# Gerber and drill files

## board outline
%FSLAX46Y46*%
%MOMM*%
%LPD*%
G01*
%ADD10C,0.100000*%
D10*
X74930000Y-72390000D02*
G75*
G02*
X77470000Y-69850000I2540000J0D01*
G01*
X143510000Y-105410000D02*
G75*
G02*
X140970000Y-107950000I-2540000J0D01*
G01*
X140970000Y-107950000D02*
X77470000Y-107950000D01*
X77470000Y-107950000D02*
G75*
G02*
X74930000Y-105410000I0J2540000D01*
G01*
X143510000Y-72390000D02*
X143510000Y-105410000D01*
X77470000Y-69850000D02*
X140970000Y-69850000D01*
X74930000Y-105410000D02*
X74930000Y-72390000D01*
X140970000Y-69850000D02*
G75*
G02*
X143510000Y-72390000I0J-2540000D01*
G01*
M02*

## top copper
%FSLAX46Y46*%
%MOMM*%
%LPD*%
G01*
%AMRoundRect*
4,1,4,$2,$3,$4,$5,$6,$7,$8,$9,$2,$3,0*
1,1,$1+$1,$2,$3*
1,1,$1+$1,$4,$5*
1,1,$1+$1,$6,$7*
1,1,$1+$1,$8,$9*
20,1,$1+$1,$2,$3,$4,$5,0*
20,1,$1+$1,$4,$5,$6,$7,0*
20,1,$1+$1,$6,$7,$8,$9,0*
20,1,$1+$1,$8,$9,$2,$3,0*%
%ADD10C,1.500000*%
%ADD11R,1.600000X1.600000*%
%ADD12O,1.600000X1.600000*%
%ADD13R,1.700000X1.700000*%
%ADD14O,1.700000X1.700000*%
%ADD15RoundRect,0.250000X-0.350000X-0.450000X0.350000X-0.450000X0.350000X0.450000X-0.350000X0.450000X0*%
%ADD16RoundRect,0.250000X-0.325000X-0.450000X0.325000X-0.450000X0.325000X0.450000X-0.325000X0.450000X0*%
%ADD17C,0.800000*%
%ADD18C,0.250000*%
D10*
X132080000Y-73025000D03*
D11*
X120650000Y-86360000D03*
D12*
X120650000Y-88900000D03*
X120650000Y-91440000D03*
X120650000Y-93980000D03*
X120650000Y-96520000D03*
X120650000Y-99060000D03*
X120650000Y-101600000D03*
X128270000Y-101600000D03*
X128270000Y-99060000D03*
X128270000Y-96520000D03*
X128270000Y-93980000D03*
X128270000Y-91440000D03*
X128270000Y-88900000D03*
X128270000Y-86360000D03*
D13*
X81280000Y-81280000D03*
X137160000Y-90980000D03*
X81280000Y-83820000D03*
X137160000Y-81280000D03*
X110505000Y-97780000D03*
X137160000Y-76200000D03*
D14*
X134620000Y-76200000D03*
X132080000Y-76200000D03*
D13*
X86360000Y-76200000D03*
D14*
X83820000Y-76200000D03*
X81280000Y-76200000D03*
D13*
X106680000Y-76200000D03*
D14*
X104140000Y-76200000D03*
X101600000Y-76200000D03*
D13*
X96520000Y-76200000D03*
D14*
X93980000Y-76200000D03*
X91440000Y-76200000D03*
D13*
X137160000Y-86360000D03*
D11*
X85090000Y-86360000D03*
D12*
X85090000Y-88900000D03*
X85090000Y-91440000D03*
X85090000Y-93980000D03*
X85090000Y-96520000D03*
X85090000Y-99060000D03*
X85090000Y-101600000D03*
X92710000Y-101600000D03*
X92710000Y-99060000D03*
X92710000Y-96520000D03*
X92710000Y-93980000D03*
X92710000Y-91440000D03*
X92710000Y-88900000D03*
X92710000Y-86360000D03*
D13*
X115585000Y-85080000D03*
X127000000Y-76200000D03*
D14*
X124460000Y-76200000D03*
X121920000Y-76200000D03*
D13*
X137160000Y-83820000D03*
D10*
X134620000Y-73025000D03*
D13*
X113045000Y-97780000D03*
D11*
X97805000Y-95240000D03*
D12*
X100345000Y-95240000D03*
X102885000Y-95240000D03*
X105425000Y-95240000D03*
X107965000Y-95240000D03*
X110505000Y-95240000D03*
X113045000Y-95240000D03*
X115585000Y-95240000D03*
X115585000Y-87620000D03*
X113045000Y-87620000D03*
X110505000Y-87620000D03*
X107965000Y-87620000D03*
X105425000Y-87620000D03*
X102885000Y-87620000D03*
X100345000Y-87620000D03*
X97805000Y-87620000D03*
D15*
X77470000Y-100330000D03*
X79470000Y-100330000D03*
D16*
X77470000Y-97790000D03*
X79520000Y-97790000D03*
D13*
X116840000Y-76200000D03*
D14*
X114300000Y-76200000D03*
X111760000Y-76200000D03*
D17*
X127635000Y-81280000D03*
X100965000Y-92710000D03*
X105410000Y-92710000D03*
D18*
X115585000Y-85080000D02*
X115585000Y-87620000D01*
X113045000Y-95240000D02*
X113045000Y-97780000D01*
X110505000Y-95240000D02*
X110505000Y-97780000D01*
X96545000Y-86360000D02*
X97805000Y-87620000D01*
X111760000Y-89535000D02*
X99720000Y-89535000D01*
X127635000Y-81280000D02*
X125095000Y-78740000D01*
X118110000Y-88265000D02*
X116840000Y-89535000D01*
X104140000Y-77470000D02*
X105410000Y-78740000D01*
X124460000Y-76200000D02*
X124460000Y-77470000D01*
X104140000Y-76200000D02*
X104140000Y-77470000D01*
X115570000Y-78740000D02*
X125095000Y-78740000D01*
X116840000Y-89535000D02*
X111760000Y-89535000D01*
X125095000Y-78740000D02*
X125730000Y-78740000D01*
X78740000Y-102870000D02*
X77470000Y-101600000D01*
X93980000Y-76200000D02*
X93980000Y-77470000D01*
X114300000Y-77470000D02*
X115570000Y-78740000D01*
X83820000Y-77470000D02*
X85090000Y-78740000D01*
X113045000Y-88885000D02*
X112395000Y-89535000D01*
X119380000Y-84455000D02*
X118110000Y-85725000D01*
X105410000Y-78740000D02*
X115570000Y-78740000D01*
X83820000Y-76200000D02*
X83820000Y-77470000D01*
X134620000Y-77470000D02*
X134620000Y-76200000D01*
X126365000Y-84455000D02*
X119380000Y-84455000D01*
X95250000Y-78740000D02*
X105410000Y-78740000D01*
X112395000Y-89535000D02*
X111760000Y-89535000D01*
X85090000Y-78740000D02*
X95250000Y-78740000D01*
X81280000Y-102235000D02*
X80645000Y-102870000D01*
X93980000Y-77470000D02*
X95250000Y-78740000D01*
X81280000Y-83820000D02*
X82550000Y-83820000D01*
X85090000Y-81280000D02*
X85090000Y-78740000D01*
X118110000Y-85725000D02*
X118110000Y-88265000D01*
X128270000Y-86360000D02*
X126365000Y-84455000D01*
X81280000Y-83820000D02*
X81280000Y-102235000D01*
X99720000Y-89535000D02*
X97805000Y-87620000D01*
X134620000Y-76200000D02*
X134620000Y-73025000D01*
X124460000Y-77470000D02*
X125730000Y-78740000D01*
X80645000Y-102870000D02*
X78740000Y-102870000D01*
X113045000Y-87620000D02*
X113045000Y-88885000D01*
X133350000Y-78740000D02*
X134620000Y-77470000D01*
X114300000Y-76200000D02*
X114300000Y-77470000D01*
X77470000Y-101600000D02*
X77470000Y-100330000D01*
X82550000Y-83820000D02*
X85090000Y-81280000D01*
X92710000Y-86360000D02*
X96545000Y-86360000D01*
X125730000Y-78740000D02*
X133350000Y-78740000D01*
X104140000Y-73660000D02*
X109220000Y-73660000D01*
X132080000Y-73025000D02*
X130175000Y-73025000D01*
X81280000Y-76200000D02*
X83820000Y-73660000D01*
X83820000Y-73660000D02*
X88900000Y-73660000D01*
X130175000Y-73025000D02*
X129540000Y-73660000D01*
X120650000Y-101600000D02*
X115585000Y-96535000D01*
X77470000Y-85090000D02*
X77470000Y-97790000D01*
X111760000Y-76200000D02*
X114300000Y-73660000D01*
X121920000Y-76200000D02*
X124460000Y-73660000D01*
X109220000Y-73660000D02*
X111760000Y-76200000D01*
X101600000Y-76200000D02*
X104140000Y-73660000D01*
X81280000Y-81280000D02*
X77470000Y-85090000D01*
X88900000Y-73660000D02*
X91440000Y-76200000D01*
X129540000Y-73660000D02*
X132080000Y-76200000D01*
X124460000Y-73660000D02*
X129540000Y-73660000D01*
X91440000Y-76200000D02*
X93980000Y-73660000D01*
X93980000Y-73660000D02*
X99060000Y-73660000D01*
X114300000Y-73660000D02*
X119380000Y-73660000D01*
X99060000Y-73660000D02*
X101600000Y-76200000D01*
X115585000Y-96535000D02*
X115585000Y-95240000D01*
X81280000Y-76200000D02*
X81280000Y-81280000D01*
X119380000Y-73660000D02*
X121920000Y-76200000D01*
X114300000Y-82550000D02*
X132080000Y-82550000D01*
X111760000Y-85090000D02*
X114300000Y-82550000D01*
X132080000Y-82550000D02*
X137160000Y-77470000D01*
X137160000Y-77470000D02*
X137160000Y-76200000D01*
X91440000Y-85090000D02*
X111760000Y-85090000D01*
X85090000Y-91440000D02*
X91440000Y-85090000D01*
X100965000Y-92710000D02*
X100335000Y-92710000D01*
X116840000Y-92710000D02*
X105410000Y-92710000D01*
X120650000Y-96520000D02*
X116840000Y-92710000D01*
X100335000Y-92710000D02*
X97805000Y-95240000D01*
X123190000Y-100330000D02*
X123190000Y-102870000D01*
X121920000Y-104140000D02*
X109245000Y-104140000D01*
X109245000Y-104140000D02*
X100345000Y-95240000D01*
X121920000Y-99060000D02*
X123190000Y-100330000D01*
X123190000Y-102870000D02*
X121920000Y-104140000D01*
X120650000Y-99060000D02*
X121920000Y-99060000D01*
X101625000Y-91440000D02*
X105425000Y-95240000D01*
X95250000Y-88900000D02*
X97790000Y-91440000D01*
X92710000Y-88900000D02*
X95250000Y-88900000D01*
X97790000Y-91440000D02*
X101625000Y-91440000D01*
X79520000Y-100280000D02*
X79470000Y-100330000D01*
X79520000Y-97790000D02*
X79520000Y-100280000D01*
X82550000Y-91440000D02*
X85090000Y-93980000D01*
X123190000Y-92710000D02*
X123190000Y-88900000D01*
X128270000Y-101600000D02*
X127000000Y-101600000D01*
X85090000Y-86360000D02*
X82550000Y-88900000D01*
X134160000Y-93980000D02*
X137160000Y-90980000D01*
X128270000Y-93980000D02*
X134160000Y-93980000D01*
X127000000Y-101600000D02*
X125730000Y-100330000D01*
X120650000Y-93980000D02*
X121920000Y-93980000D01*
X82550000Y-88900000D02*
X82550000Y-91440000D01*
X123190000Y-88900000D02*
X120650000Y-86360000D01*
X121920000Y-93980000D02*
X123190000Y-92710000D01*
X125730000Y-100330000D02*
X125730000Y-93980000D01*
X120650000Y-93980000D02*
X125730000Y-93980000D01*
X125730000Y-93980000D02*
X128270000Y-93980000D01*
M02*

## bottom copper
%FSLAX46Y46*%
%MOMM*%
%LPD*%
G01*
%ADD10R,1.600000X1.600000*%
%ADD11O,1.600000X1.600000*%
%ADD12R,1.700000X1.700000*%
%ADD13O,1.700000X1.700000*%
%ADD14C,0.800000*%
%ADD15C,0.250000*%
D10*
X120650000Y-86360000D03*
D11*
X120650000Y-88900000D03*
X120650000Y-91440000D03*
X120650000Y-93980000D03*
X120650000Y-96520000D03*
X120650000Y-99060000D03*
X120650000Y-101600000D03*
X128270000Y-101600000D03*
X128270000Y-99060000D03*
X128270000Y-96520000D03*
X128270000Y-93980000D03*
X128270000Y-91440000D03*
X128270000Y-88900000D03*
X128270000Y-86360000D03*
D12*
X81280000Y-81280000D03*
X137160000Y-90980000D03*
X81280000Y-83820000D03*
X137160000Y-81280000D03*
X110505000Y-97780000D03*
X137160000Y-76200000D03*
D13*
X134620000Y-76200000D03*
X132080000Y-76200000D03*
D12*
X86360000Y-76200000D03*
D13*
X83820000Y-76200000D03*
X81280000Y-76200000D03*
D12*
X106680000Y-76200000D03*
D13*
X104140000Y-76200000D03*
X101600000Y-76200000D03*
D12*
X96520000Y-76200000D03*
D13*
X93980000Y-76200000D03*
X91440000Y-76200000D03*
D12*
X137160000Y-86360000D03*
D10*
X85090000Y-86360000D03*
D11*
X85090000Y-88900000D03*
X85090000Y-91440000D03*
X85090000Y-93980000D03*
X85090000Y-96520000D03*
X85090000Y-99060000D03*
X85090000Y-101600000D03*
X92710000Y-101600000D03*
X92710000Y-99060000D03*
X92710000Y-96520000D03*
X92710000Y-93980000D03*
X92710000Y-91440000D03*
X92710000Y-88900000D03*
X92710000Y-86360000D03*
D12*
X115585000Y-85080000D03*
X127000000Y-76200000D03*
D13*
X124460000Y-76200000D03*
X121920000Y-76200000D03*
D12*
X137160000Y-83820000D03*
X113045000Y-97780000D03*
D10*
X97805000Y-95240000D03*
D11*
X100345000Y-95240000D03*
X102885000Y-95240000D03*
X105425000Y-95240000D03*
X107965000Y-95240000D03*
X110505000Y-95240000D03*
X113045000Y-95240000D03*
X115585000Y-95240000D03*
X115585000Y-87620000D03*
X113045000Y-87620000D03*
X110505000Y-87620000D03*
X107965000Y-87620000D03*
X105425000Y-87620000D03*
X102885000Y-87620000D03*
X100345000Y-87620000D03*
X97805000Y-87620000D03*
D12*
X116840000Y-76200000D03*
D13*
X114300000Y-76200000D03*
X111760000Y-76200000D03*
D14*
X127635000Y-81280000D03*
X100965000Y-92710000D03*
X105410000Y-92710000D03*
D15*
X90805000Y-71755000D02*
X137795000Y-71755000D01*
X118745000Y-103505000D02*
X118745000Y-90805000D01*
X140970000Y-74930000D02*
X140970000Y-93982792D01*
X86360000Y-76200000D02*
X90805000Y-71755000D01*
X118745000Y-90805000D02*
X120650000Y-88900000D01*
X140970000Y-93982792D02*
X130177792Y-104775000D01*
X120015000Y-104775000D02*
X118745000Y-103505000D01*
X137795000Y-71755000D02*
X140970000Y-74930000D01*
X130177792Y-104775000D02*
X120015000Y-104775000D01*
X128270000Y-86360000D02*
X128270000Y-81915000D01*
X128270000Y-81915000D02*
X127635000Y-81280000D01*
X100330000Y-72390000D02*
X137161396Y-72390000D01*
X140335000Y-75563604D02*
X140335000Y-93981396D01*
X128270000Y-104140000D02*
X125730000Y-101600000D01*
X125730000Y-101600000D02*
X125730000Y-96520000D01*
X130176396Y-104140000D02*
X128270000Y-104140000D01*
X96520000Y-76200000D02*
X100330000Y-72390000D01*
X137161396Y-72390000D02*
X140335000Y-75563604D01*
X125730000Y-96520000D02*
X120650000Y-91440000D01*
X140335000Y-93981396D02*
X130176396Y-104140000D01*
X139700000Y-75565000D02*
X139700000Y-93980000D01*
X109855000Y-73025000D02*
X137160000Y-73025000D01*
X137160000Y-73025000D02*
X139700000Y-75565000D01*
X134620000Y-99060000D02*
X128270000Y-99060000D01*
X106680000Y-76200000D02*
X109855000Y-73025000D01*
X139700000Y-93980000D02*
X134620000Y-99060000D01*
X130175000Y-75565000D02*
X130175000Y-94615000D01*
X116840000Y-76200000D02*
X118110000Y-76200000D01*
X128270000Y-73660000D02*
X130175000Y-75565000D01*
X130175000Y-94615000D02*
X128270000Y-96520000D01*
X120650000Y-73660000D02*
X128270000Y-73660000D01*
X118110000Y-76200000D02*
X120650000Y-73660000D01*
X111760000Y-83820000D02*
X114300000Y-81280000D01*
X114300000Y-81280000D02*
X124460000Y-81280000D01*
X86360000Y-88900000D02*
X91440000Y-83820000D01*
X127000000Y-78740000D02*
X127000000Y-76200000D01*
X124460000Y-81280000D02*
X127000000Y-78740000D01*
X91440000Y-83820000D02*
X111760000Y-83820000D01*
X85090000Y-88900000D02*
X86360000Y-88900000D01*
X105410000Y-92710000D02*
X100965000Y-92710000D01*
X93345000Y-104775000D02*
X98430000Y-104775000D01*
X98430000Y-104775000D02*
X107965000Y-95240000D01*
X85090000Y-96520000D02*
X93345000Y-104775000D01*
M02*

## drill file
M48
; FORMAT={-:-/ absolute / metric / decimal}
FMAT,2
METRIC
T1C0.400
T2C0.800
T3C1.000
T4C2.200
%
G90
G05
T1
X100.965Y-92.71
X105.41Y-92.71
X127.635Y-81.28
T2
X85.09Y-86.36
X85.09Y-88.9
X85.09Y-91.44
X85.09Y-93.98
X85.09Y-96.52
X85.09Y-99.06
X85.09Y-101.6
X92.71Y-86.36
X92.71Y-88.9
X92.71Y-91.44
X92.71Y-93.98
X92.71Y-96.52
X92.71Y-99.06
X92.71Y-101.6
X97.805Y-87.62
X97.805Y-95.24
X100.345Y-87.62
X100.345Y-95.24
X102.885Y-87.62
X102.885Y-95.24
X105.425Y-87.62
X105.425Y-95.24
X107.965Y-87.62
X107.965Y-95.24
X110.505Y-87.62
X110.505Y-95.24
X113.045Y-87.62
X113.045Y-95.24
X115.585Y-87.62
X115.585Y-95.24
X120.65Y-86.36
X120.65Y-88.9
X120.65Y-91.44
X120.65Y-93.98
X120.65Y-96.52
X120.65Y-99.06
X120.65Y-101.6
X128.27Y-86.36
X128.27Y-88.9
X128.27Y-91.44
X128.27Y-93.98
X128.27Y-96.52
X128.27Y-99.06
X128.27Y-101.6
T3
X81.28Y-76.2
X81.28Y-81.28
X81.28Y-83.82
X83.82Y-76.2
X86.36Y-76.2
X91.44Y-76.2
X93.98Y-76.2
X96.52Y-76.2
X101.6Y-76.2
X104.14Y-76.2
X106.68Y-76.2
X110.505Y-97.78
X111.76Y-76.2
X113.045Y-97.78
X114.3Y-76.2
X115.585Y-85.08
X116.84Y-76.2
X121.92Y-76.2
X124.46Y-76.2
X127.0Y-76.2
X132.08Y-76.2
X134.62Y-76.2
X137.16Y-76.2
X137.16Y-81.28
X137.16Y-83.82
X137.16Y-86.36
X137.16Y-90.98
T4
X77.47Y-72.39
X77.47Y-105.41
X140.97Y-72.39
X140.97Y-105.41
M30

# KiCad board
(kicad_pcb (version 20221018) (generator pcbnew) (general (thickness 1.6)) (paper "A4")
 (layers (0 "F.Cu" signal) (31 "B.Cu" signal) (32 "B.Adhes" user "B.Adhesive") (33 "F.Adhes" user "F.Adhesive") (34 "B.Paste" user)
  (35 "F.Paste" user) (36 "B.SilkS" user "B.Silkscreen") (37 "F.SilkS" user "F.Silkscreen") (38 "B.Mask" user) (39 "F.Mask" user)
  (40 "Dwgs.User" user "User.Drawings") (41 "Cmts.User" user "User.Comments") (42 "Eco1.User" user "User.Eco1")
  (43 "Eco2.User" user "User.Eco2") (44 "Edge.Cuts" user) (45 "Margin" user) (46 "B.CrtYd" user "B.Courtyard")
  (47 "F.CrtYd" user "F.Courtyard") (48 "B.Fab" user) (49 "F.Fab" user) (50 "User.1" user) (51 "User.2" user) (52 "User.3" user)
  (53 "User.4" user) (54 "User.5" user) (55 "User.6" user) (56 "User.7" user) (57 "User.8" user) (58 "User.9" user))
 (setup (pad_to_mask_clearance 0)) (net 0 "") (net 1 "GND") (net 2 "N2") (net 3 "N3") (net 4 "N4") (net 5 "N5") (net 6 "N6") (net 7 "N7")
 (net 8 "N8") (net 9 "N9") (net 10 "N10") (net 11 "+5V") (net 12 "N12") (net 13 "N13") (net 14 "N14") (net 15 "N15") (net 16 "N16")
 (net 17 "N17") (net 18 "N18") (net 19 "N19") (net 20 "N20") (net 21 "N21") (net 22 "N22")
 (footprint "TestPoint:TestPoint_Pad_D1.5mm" (layer "F.Cu") (at 132.08 73.025)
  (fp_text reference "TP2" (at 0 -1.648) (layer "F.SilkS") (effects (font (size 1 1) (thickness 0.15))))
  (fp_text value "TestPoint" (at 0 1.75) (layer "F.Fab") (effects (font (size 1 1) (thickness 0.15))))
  (pad "1" smd circle (at 0 0) (size 1.5 1.5) (layers "F.Cu" "F.Mask") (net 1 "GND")))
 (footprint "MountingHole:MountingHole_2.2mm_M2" (layer "F.Cu") (at 77.47 72.39)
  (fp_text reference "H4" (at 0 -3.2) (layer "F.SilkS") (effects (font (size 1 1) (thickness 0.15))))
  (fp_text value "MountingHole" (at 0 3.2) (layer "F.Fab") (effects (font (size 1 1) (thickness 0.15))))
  (pad "" np_thru_hole circle (at 0 0) (size 2.2 2.2) (drill 2.2) (layers "*.Cu" "*.Mask")))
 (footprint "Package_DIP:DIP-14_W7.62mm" (layer "F.Cu") (at 120.65 86.36)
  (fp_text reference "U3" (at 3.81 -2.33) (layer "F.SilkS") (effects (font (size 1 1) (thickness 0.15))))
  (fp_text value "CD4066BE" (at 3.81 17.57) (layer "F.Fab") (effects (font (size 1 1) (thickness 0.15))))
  (pad "1" thru_hole rect (at 0 0) (size 1.6 1.6) (drill 0.8) (layers "*.Cu" "*.Mask") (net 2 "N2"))
  (pad "2" thru_hole oval (at 0 2.54) (size 1.6 1.6) (drill 0.8) (layers "*.Cu" "*.Mask") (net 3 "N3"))
  (pad "3" thru_hole oval (at 0 5.08) (size 1.6 1.6) (drill 0.8) (layers "*.Cu" "*.Mask") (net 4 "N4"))
  (pad "4" thru_hole oval (at 0 7.62) (size 1.6 1.6) (drill 0.8) (layers "*.Cu" "*.Mask") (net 2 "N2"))
  (pad "5" thru_hole oval (at 0 10.16) (size 1.6 1.6) (drill 0.8) (layers "*.Cu" "*.Mask") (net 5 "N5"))
  (pad "6" thru_hole oval (at 0 12.7) (size 1.6 1.6) (drill 0.8) (layers "*.Cu" "*.Mask") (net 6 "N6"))
  (pad "7" thru_hole oval (at 0 15.24) (size 1.6 1.6) (drill 0.8) (layers "*.Cu" "*.Mask") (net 1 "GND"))
  (pad "8" thru_hole oval (at 7.62 15.24) (size 1.6 1.6) (drill 0.8) (layers "*.Cu" "*.Mask") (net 2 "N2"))
  (pad "9" thru_hole oval (at 7.62 12.7) (size 1.6 1.6) (drill 0.8) (layers "*.Cu" "*.Mask") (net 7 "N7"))
  (pad "10" thru_hole oval (at 7.62 10.16) (size 1.6 1.6) (drill 0.8) (layers "*.Cu" "*.Mask") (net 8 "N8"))
  (pad "11" thru_hole oval (at 7.62 7.62) (size 1.6 1.6) (drill 0.8) (layers "*.Cu" "*.Mask") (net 2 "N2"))
  (pad "12" thru_hole oval (at 7.62 5.08) (size 1.6 1.6) (drill 0.8) (layers "*.Cu" "*.Mask") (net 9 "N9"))
  (pad "13" thru_hole oval (at 7.62 2.54) (size 1.6 1.6) (drill 0.8) (layers "*.Cu" "*.Mask") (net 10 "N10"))
  (pad "14" thru_hole oval (at 7.62 0) (size 1.6 1.6) (drill 0.8) (layers "*.Cu" "*.Mask") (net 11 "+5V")))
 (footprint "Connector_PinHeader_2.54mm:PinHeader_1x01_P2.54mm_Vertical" (layer "F.Cu") (at 81.28 81.28)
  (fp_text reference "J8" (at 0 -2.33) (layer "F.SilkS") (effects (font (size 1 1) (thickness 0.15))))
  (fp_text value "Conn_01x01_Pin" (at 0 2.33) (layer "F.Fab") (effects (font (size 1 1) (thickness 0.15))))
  (pad "1" thru_hole rect (at 0 0) (size 1.7 1.7) (drill 1) (layers "*.Cu" "*.Mask") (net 1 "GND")))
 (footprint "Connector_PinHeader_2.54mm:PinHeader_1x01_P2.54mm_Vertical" (layer "F.Cu") (at 137.16 90.98)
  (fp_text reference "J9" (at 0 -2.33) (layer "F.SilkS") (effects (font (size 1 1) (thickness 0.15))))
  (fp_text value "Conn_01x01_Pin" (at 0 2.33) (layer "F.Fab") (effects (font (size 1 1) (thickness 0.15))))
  (pad "1" thru_hole rect (at 0 0) (size 1.7 1.7) (drill 1) (layers "*.Cu" "*.Mask") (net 2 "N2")))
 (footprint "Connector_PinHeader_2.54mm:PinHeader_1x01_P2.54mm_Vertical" (layer "F.Cu") (at 81.28 83.82)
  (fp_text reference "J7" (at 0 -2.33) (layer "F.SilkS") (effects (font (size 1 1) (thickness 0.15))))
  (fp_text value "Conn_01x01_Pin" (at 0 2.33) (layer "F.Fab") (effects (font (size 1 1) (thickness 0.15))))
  (pad "1" thru_hole rect (at 0 0) (size 1.7 1.7) (drill 1) (layers "*.Cu" "*.Mask") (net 11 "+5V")))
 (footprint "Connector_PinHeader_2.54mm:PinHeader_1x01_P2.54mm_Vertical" (layer "F.Cu") (at 137.16 81.28 90)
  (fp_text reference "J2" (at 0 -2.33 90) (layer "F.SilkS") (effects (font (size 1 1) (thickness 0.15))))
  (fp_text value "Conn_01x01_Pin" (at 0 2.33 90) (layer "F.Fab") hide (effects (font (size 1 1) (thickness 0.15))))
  (pad "1" thru_hole rect (at 0 0 90) (size 1.7 1.7) (drill 1) (layers "*.Cu" "*.Mask") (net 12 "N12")))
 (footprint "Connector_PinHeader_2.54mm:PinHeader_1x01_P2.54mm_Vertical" (layer "F.Cu") (at 110.505 97.78)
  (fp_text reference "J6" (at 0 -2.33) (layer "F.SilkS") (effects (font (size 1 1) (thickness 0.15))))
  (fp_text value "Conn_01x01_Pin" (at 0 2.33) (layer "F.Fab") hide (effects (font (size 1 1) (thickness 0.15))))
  (pad "1" thru_hole rect (at 0 0) (size 1.7 1.7) (drill 1) (layers "*.Cu" "*.Mask") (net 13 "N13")))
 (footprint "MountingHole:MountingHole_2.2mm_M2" (layer "F.Cu") (at 140.97 72.39)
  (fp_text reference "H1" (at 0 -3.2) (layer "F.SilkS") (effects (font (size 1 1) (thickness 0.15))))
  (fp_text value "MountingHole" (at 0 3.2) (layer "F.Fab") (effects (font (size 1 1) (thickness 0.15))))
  (pad "" np_thru_hole circle (at 0 0) (size 2.2 2.2) (drill 2.2) (layers "*.Cu" "*.Mask")))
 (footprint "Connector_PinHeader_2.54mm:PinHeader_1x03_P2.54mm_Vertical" (layer "F.Cu") (at 137.16 76.2 -90)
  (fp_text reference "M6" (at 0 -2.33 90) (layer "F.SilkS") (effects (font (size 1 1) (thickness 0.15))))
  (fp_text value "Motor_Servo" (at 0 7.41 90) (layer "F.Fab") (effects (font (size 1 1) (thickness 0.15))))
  (pad "1" thru_hole rect (at 0 0 270) (size 1.7 1.7) (drill 1) (layers "*.Cu" "*.Mask") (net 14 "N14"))
  (pad "2" thru_hole oval (at 0 2.54 270) (size 1.7 1.7) (drill 1) (layers "*.Cu" "*.Mask") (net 11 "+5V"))
  (pad "3" thru_hole oval (at 0 5.08 270) (size 1.7 1.7) (drill 1) (layers "*.Cu" "*.Mask") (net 1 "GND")))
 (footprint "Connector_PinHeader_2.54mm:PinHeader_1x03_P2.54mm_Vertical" (layer "F.Cu") (at 86.36 76.2 -90)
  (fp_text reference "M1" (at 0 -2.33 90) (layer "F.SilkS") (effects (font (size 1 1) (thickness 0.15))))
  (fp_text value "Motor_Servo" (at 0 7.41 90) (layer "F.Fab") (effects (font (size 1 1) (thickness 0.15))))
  (pad "1" thru_hole rect (at 0 0 270) (size 1.7 1.7) (drill 1) (layers "*.Cu" "*.Mask") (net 3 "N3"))
  (pad "2" thru_hole oval (at 0 2.54 270) (size 1.7 1.7) (drill 1) (layers "*.Cu" "*.Mask") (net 11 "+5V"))
  (pad "3" thru_hole oval (at 0 5.08 270) (size 1.7 1.7) (drill 1) (layers "*.Cu" "*.Mask") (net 1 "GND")))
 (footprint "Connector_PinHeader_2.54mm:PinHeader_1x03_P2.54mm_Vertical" (layer "F.Cu") (at 106.68 76.2 -90)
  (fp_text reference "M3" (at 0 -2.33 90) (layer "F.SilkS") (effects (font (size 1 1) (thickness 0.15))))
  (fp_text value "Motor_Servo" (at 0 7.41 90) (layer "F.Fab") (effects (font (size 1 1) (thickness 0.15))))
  (pad "1" thru_hole rect (at 0 0 270) (size 1.7 1.7) (drill 1) (layers "*.Cu" "*.Mask") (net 7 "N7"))
  (pad "2" thru_hole oval (at 0 2.54 270) (size 1.7 1.7) (drill 1) (layers "*.Cu" "*.Mask") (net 11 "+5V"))
  (pad "3" thru_hole oval (at 0 5.08 270) (size 1.7 1.7) (drill 1) (layers "*.Cu" "*.Mask") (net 1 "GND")))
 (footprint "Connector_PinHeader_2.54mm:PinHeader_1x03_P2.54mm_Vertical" (layer "F.Cu") (at 96.52 76.2 -90)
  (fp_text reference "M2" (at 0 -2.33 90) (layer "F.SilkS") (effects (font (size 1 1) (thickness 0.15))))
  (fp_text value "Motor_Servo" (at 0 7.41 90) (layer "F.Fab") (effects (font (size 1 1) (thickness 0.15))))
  (pad "1" thru_hole rect (at 0 0 270) (size 1.7 1.7) (drill 1) (layers "*.Cu" "*.Mask") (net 4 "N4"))
  (pad "2" thru_hole oval (at 0 2.54 270) (size 1.7 1.7) (drill 1) (layers "*.Cu" "*.Mask") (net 11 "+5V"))
  (pad "3" thru_hole oval (at 0 5.08 270) (size 1.7 1.7) (drill 1) (layers "*.Cu" "*.Mask") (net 1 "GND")))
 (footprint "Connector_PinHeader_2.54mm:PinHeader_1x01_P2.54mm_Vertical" (layer "F.Cu") (at 137.16 86.36 90)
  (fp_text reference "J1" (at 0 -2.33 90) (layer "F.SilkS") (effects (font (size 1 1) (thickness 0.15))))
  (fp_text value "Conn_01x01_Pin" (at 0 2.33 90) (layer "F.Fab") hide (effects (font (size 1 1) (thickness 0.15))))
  (pad "1" thru_hole rect (at 0 0 90) (size 1.7 1.7) (drill 1) (layers "*.Cu" "*.Mask") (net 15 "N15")))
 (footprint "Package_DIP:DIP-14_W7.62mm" (layer "F.Cu") (at 85.09 86.36)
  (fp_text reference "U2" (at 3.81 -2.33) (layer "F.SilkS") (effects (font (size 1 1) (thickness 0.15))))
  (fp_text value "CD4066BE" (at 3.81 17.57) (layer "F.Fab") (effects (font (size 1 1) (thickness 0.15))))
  (pad "1" thru_hole rect (at 0 0) (size 1.6 1.6) (drill 0.8) (layers "*.Cu" "*.Mask") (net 2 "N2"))
  (pad "2" thru_hole oval (at 0 2.54) (size 1.6 1.6) (drill 0.8) (layers "*.Cu" "*.Mask") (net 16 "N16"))
  (pad "3" thru_hole oval (at 0 5.08) (size 1.6 1.6) (drill 0.8) (layers "*.Cu" "*.Mask") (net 14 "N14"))
  (pad "4" thru_hole oval (at 0 7.62) (size 1.6 1.6) (drill 0.8) (layers "*.Cu" "*.Mask") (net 2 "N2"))
  (pad "5" thru_hole oval (at 0 10.16) (size 1.6 1.6) (drill 0.8) (layers "*.Cu" "*.Mask") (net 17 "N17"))
  (pad "6" thru_hole oval (at 0 12.7) (size 1.6 1.6) (drill 0.8) (layers "*.Cu" "*.Mask"))
  (pad "7" thru_hole oval (at 0 15.24) (size 1.6 1.6) (drill 0.8) (layers "*.Cu" "*.Mask") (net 1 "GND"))
  (pad "8" thru_hole oval (at 7.62 15.24) (size 1.6 1.6) (drill 0.8) (layers "*.Cu" "*.Mask"))
  (pad "9" thru_hole oval (at 7.62 12.7) (size 1.6 1.6) (drill 0.8) (layers "*.Cu" "*.Mask"))
  (pad "10" thru_hole oval (at 7.62 10.16) (size 1.6 1.6) (drill 0.8) (layers "*.Cu" "*.Mask"))
  (pad "11" thru_hole oval (at 7.62 7.62) (size 1.6 1.6) (drill 0.8) (layers "*.Cu" "*.Mask"))
  (pad "12" thru_hole oval (at 7.62 5.08) (size 1.6 1.6) (drill 0.8) (layers "*.Cu" "*.Mask"))
  (pad "13" thru_hole oval (at 7.62 2.54) (size 1.6 1.6) (drill 0.8) (layers "*.Cu" "*.Mask") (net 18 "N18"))
  (pad "14" thru_hole oval (at 7.62 0) (size 1.6 1.6) (drill 0.8) (layers "*.Cu" "*.Mask") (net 11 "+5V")))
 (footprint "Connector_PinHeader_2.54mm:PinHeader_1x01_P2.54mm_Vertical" (layer "F.Cu") (at 115.585 85.08)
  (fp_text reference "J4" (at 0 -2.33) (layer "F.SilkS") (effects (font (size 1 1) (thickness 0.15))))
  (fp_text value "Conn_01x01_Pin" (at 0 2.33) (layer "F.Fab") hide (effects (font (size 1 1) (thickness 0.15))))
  (pad "1" thru_hole rect (at 0 0) (size 1.7 1.7) (drill 1) (layers "*.Cu" "*.Mask") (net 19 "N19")))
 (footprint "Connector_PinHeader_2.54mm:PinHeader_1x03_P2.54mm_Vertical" (layer "F.Cu") (at 127 76.2 -90)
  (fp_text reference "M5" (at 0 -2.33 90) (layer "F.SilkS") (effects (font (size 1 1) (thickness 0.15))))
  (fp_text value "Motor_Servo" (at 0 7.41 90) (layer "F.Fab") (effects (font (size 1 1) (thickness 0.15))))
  (pad "1" thru_hole rect (at 0 0 270) (size 1.7 1.7) (drill 1) (layers "*.Cu" "*.Mask") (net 16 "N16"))
  (pad "2" thru_hole oval (at 0 2.54 270) (size 1.7 1.7) (drill 1) (layers "*.Cu" "*.Mask") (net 11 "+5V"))
  (pad "3" thru_hole oval (at 0 5.08 270) (size 1.7 1.7) (drill 1) (layers "*.Cu" "*.Mask") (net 1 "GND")))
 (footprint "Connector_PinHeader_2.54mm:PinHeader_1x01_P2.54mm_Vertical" (layer "F.Cu") (at 137.16 83.82 90)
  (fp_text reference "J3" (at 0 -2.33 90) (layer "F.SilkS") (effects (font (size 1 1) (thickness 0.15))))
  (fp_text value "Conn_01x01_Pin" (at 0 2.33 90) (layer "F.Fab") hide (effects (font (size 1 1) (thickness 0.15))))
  (pad "1" thru_hole rect (at 0 0 90) (size 1.7 1.7) (drill 1) (layers "*.Cu" "*.Mask") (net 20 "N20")))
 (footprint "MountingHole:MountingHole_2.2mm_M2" (layer "F.Cu") (at 140.97 105.41)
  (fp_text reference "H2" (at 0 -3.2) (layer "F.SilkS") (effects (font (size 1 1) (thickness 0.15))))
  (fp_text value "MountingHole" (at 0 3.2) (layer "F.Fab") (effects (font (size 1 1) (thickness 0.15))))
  (pad "" np_thru_hole circle (at 0 0) (size 2.2 2.2) (drill 2.2) (layers "*.Cu" "*.Mask")))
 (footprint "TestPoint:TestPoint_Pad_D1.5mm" (layer "F.Cu") (at 134.62 73.025)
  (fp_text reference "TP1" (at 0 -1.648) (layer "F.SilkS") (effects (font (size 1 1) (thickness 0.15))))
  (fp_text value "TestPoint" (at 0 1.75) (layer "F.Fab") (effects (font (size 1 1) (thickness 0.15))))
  (pad "1" smd circle (at 0 0) (size 1.5 1.5) (layers "F.Cu" "F.Mask") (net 11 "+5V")))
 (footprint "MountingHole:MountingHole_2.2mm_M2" (layer "F.Cu") (at 77.47 105.41)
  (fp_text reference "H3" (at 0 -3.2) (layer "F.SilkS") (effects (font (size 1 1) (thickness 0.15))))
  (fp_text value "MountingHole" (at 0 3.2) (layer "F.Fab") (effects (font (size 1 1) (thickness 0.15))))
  (pad "" np_thru_hole circle (at 0 0) (size 2.2 2.2) (drill 2.2) (layers "*.Cu" "*.Mask")))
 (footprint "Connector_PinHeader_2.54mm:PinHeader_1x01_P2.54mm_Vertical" (layer "F.Cu") (at 113.045 97.78)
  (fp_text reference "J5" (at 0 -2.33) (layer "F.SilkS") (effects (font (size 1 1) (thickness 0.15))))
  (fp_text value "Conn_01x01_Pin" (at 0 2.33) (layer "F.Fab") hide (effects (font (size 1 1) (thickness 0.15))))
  (pad "1" thru_hole rect (at 0 0) (size 1.7 1.7) (drill 1) (layers "*.Cu" "*.Mask") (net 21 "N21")))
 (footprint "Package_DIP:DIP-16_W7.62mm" (layer "F.Cu") (at 97.805 95.24 90)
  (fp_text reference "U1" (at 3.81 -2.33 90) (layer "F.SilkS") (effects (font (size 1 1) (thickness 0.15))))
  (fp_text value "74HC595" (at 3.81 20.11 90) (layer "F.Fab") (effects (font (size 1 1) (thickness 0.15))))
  (pad "1" thru_hole rect (at 0 0 90) (size 1.6 1.6) (drill 0.8) (layers "*.Cu" "*.Mask") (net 5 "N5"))
  (pad "2" thru_hole oval (at 0 2.54 90) (size 1.6 1.6) (drill 0.8) (layers "*.Cu" "*.Mask") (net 6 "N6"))
  (pad "3" thru_hole oval (at 0 5.08 90) (size 1.6 1.6) (drill 0.8) (layers "*.Cu" "*.Mask") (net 9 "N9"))
  (pad "4" thru_hole oval (at 0 7.62 90) (size 1.6 1.6) (drill 0.8) (layers "*.Cu" "*.Mask") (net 18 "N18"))
  (pad "5" thru_hole oval (at 0 10.16 90) (size 1.6 1.6) (drill 0.8) (layers "*.Cu" "*.Mask") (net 17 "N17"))
  (pad "6" thru_hole oval (at 0 12.7 90) (size 1.6 1.6) (drill 0.8) (layers "*.Cu" "*.Mask") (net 13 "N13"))
  (pad "7" thru_hole oval (at 0 15.24 90) (size 1.6 1.6) (drill 0.8) (layers "*.Cu" "*.Mask") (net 21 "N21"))
  (pad "8" thru_hole oval (at 0 17.78 90) (size 1.6 1.6) (drill 0.8) (layers "*.Cu" "*.Mask") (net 1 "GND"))
  (pad "9" thru_hole oval (at 7.62 17.78 90) (size 1.6 1.6) (drill 0.8) (layers "*.Cu" "*.Mask") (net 19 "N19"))
  (pad "10" thru_hole oval (at 7.62 15.24 90) (size 1.6 1.6) (drill 0.8) (layers "*.Cu" "*.Mask") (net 11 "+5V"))
  (pad "11" thru_hole oval (at 7.62 12.7 90) (size 1.6 1.6) (drill 0.8) (layers "*.Cu" "*.Mask") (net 12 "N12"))
  (pad "12" thru_hole oval (at 7.62 10.16 90) (size 1.6 1.6) (drill 0.8) (layers "*.Cu" "*.Mask") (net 20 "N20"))
  (pad "13" thru_hole oval (at 7.62 7.62 90) (size 1.6 1.6) (drill 0.8) (layers "*.Cu" "*.Mask") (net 1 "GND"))
  (pad "14" thru_hole oval (at 7.62 5.08 90) (size 1.6 1.6) (drill 0.8) (layers "*.Cu" "*.Mask") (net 15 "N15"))
  (pad "15" thru_hole oval (at 7.62 2.54 90) (size 1.6 1.6) (drill 0.8) (layers "*.Cu" "*.Mask") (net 10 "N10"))
  (pad "16" thru_hole oval (at 7.62 0 90) (size 1.6 1.6) (drill 0.8) (layers "*.Cu" "*.Mask") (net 11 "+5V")))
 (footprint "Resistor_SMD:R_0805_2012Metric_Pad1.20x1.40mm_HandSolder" (layer "F.Cu") (at 78.47 100.33)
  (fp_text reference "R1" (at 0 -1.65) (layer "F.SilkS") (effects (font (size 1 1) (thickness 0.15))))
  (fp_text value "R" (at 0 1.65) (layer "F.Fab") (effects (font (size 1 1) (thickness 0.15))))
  (pad "1" smd roundrect (at -1 0) (size 1.2 1.4) (layers "F.Cu" "F.Paste" "F.Mask") (roundrect_rratio 0.208333) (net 11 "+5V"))
  (pad "2" smd roundrect (at 1 0) (size 1.2 1.4) (layers "F.Cu" "F.Paste" "F.Mask") (roundrect_rratio 0.208333) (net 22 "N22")))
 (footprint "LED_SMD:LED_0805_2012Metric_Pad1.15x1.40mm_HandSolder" (layer "F.Cu") (at 78.495 97.79)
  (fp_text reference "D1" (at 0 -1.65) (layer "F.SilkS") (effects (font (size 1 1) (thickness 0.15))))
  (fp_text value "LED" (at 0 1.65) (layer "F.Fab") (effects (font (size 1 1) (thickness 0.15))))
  (pad "1" smd roundrect (at -1.025 0) (size 1.15 1.4) (layers "F.Cu" "F.Paste" "F.Mask") (roundrect_rratio 0.217391) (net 1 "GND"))
  (pad "2" smd roundrect (at 1.025 0) (size 1.15 1.4) (layers "F.Cu" "F.Paste" "F.Mask") (roundrect_rratio 0.217391) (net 22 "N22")))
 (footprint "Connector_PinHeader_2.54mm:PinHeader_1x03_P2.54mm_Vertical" (layer "F.Cu") (at 116.84 76.2 -90)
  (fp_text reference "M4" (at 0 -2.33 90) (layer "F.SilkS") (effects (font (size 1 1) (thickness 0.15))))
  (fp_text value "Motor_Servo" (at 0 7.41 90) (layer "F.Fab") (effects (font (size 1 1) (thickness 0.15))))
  (pad "1" thru_hole rect (at 0 0 270) (size 1.7 1.7) (drill 1) (layers "*.Cu" "*.Mask") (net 8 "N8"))
  (pad "2" thru_hole oval (at 0 2.54 270) (size 1.7 1.7) (drill 1) (layers "*.Cu" "*.Mask") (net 11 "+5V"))
  (pad "3" thru_hole oval (at 0 5.08 270) (size 1.7 1.7) (drill 1) (layers "*.Cu" "*.Mask") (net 1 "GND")))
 (gr_arc (start 74.93 72.39) (mid 75.673949 70.593949) (end 77.47 69.85) (stroke (width 0.1) (type default)) (layer "Edge.Cuts"))
 (gr_arc (start 143.51 105.41) (mid 142.766051 107.206051) (end 140.97 107.95) (stroke (width 0.1) (type default)) (layer "Edge.Cuts"))
 (gr_line (start 140.97 107.95) (end 77.47 107.95) (stroke (width 0.1) (type default)) (layer "Edge.Cuts"))
 (gr_arc (start 77.47 107.95) (mid 75.673949 107.206051) (end 74.93 105.41) (stroke (width 0.1) (type default)) (layer "Edge.Cuts"))
 (gr_line (start 143.51 72.39) (end 143.51 105.41) (stroke (width 0.1) (type default)) (layer "Edge.Cuts"))
 (gr_line (start 77.47 69.85) (end 140.97 69.85) (stroke (width 0.1) (type default)) (layer "Edge.Cuts"))
 (gr_line (start 74.93 105.41) (end 74.93 72.39) (stroke (width 0.1) (type default)) (layer "Edge.Cuts"))
 (gr_arc (start 140.97 69.85) (mid 142.766051 70.593949) (end 143.51 72.39) (stroke (width 0.1) (type default)) (layer "Edge.Cuts"))
 (segment (start 115.585 85.08) (end 115.585 87.62) (width 0.25) (layer "F.Cu") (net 19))
 (segment (start 113.045 95.24) (end 113.045 97.78) (width 0.25) (layer "F.Cu") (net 21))
 (segment (start 110.505 95.24) (end 110.505 97.78) (width 0.25) (layer "F.Cu") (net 13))
 (segment (start 90.805 71.755) (end 137.795 71.755) (width 0.25) (layer "B.Cu") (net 3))
 (segment (start 118.745 103.505) (end 118.745 90.805) (width 0.25) (layer "B.Cu") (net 3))
 (segment (start 140.97 74.93) (end 140.97 93.982792) (width 0.25) (layer "B.Cu") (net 3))
 (segment (start 86.36 76.2) (end 90.805 71.755) (width 0.25) (layer "B.Cu") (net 3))
 (segment (start 118.745 90.805) (end 120.65 88.9) (width 0.25) (layer "B.Cu") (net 3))
 (segment (start 140.97 93.982792) (end 130.177792 104.775) (width 0.25) (layer "B.Cu") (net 3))
 (segment (start 120.015 104.775) (end 118.745 103.505) (width 0.25) (layer "B.Cu") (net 3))
 (segment (start 137.795 71.755) (end 140.97 74.93) (width 0.25) (layer "B.Cu") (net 3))
 (segment (start 130.177792 104.775) (end 120.015 104.775) (width 0.25) (layer "B.Cu") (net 3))
 (segment (start 96.545 86.36) (end 97.805 87.62) (width 0.25) (layer "F.Cu") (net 11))
 (segment (start 111.76 89.535) (end 99.72 89.535) (width 0.25) (layer "F.Cu") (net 11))
 (segment (start 127.635 81.28) (end 125.095 78.74) (width 0.25) (layer "F.Cu") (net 11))
 (segment (start 118.11 88.265) (end 116.84 89.535) (width 0.25) (layer "F.Cu") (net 11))
 (segment (start 104.14 77.47) (end 105.41 78.74) (width 0.25) (layer "F.Cu") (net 11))
 (segment (start 124.46 76.2) (end 124.46 77.47) (width 0.25) (layer "F.Cu") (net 11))
 (segment (start 104.14 76.2) (end 104.14 77.47) (width 0.25) (layer "F.Cu") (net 11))
 (segment (start 115.57 78.74) (end 125.095 78.74) (width 0.25) (layer "F.Cu") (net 11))
 (segment (start 116.84 89.535) (end 111.76 89.535) (width 0.25) (layer "F.Cu") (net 11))
 (segment (start 125.095 78.74) (end 125.73 78.74) (width 0.25) (layer "F.Cu") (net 11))
 (segment (start 78.74 102.87) (end 77.47 101.6) (width 0.25) (layer "F.Cu") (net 11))
 (segment (start 93.98 76.2) (end 93.98 77.47) (width 0.25) (layer "F.Cu") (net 11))
 (segment (start 114.3 77.47) (end 115.57 78.74) (width 0.25) (layer "F.Cu") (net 11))
 (segment (start 83.82 77.47) (end 85.09 78.74) (width 0.25) (layer "F.Cu") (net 11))
 (segment (start 113.045 88.885) (end 112.395 89.535) (width 0.25) (layer "F.Cu") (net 11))
 (segment (start 119.38 84.455) (end 118.11 85.725) (width 0.25) (layer "F.Cu") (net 11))
 (segment (start 105.41 78.74) (end 115.57 78.74) (width 0.25) (layer "F.Cu") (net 11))
 (segment (start 83.82 76.2) (end 83.82 77.47) (width 0.25) (layer "F.Cu") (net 11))
 (segment (start 134.62 77.47) (end 134.62 76.2) (width 0.25) (layer "F.Cu") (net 11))
 (segment (start 126.365 84.455) (end 119.38 84.455) (width 0.25) (layer "F.Cu") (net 11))
 (segment (start 95.25 78.74) (end 105.41 78.74) (width 0.25) (layer "F.Cu") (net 11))
 (segment (start 112.395 89.535) (end 111.76 89.535) (width 0.25) (layer "F.Cu") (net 11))
 (segment (start 85.09 78.74) (end 95.25 78.74) (width 0.25) (layer "F.Cu") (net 11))
 (segment (start 81.28 102.235) (end 80.645 102.87) (width 0.25) (layer "F.Cu") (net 11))
 (segment (start 93.98 77.47) (end 95.25 78.74) (width 0.25) (layer "F.Cu") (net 11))
 (segment (start 81.28 83.82) (end 82.55 83.82) (width 0.25) (layer "F.Cu") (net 11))
 (segment (start 85.09 81.28) (end 85.09 78.74) (width 0.25) (layer "F.Cu") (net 11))
 (segment (start 118.11 85.725) (end 118.11 88.265) (width 0.25) (layer "F.Cu") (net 11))
 (segment (start 128.27 86.36) (end 126.365 84.455) (width 0.25) (layer "F.Cu") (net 11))
 (segment (start 81.28 83.82) (end 81.28 102.235) (width 0.25) (layer "F.Cu") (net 11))
 (segment (start 99.72 89.535) (end 97.805 87.62) (width 0.25) (layer "F.Cu") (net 11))
 (segment (start 134.62 76.2) (end 134.62 73.025) (width 0.25) (layer "F.Cu") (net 11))
 (segment (start 124.46 77.47) (end 125.73 78.74) (width 0.25) (layer "F.Cu") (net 11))
 (segment (start 80.645 102.87) (end 78.74 102.87) (width 0.25) (layer "F.Cu") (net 11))
 (segment (start 113.045 87.62) (end 113.045 88.885) (width 0.25) (layer "F.Cu") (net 11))
 (segment (start 133.35 78.74) (end 134.62 77.47) (width 0.25) (layer "F.Cu") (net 11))
 (segment (start 114.3 76.2) (end 114.3 77.47) (width 0.25) (layer "F.Cu") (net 11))
 (segment (start 77.47 101.6) (end 77.47 100.33) (width 0.25) (layer "F.Cu") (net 11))
 (segment (start 82.55 83.82) (end 85.09 81.28) (width 0.25) (layer "F.Cu") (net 11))
 (segment (start 92.71 86.36) (end 96.545 86.36) (width 0.25) (layer "F.Cu") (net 11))
 (segment (start 125.73 78.74) (end 133.35 78.74) (width 0.25) (layer "F.Cu") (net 11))
 (via (at 127.635 81.28) (size 0.8) (drill 0.4) (layers "F.Cu" "B.Cu") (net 11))
 (segment (start 128.27 86.36) (end 128.27 81.915) (width 0.25) (layer "B.Cu") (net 11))
 (segment (start 128.27 81.915) (end 127.635 81.28) (width 0.25) (layer "B.Cu") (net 11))
 (segment (start 104.14 73.66) (end 109.22 73.66) (width 0.25) (layer "F.Cu") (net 1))
 (segment (start 132.08 73.025) (end 130.175 73.025) (width 0.25) (layer "F.Cu") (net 1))
 (segment (start 81.28 76.2) (end 83.82 73.66) (width 0.25) (layer "F.Cu") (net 1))
 (segment (start 83.82 73.66) (end 88.9 73.66) (width 0.25) (layer "F.Cu") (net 1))
 (segment (start 130.175 73.025) (end 129.54 73.66) (width 0.25) (layer "F.Cu") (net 1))
 (segment (start 120.65 101.6) (end 115.585 96.535) (width 0.25) (layer "F.Cu") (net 1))
 (segment (start 77.47 85.09) (end 77.47 97.79) (width 0.25) (layer "F.Cu") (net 1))
 (segment (start 111.76 76.2) (end 114.3 73.66) (width 0.25) (layer "F.Cu") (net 1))
 (segment (start 121.92 76.2) (end 124.46 73.66) (width 0.25) (layer "F.Cu") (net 1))
 (segment (start 109.22 73.66) (end 111.76 76.2) (width 0.25) (layer "F.Cu") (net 1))
 (segment (start 101.6 76.2) (end 104.14 73.66) (width 0.25) (layer "F.Cu") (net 1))
 (segment (start 81.28 81.28) (end 77.47 85.09) (width 0.25) (layer "F.Cu") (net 1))
 (segment (start 88.9 73.66) (end 91.44 76.2) (width 0.25) (layer "F.Cu") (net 1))
 (segment (start 129.54 73.66) (end 132.08 76.2) (width 0.25) (layer "F.Cu") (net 1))
 (segment (start 124.46 73.66) (end 129.54 73.66) (width 0.25) (layer "F.Cu") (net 1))
 (segment (start 91.44 76.2) (end 93.98 73.66) (width 0.25) (layer "F.Cu") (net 1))
 (segment (start 93.98 73.66) (end 99.06 73.66) (width 0.25) (layer "F.Cu") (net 1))
 (segment (start 114.3 73.66) (end 119.38 73.66) (width 0.25) (layer "F.Cu") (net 1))
 (segment (start 99.06 73.66) (end 101.6 76.2) (width 0.25) (layer "F.Cu") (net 1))
 (segment (start 115.585 96.535) (end 115.585 95.24) (width 0.25) (layer "F.Cu") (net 1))
 (segment (start 81.28 76.2) (end 81.28 81.28) (width 0.25) (layer "F.Cu") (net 1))
 (segment (start 119.38 73.66) (end 121.92 76.2) (width 0.25) (layer "F.Cu") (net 1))
 (segment (start 100.33 72.39) (end 137.161396 72.39) (width 0.25) (layer "B.Cu") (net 4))
 (segment (start 140.335 75.563604) (end 140.335 93.981396) (width 0.25) (layer "B.Cu") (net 4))
 (segment (start 128.27 104.14) (end 125.73 101.6) (width 0.25) (layer "B.Cu") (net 4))
 (segment (start 125.73 101.6) (end 125.73 96.52) (width 0.25) (layer "B.Cu") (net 4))
 (segment (start 130.176396 104.14) (end 128.27 104.14) (width 0.25) (layer "B.Cu") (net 4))
 (segment (start 96.52 76.2) (end 100.33 72.39) (width 0.25) (layer "B.Cu") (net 4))
 (segment (start 137.161396 72.39) (end 140.335 75.563604) (width 0.25) (layer "B.Cu") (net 4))
 (segment (start 125.73 96.52) (end 120.65 91.44) (width 0.25) (layer "B.Cu") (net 4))
 (segment (start 140.335 93.981396) (end 130.176396 104.14) (width 0.25) (layer "B.Cu") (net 4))
 (segment (start 139.7 75.565) (end 139.7 93.98) (width 0.25) (layer "B.Cu") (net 7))
 (segment (start 109.855 73.025) (end 137.16 73.025) (width 0.25) (layer "B.Cu") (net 7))
 (segment (start 137.16 73.025) (end 139.7 75.565) (width 0.25) (layer "B.Cu") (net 7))
 (segment (start 134.62 99.06) (end 128.27 99.06) (width 0.25) (layer "B.Cu") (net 7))
 (segment (start 106.68 76.2) (end 109.855 73.025) (width 0.25) (layer "B.Cu") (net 7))
 (segment (start 139.7 93.98) (end 134.62 99.06) (width 0.25) (layer "B.Cu") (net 7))
 (segment (start 130.175 75.565) (end 130.175 94.615) (width 0.25) (layer "B.Cu") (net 8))
 (segment (start 116.84 76.2) (end 118.11 76.2) (width 0.25) (layer "B.Cu") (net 8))
 (segment (start 128.27 73.66) (end 130.175 75.565) (width 0.25) (layer "B.Cu") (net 8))
 (segment (start 130.175 94.615) (end 128.27 96.52) (width 0.25) (layer "B.Cu") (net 8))
 (segment (start 120.65 73.66) (end 128.27 73.66) (width 0.25) (layer "B.Cu") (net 8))
 (segment (start 118.11 76.2) (end 120.65 73.66) (width 0.25) (layer "B.Cu") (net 8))
 (segment (start 111.76 83.82) (end 114.3 81.28) (width 0.25) (layer "B.Cu") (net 16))
 (segment (start 114.3 81.28) (end 124.46 81.28) (width 0.25) (layer "B.Cu") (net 16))
 (segment (start 86.36 88.9) (end 91.44 83.82) (width 0.25) (layer "B.Cu") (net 16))
 (segment (start 127 78.74) (end 127 76.2) (width 0.25) (layer "B.Cu") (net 16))
 (segment (start 124.46 81.28) (end 127 78.74) (width 0.25) (layer "B.Cu") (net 16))
 (segment (start 91.44 83.82) (end 111.76 83.82) (width 0.25) (layer "B.Cu") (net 16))
 (segment (start 85.09 88.9) (end 86.36 88.9) (width 0.25) (layer "B.Cu") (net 16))
 (segment (start 114.3 82.55) (end 132.08 82.55) (width 0.25) (layer "F.Cu") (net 14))
 (segment (start 111.76 85.09) (end 114.3 82.55) (width 0.25) (layer "F.Cu") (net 14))
 (segment (start 132.08 82.55) (end 137.16 77.47) (width 0.25) (layer "F.Cu") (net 14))
 (segment (start 137.16 77.47) (end 137.16 76.2) (width 0.25) (layer "F.Cu") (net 14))
 (segment (start 91.44 85.09) (end 111.76 85.09) (width 0.25) (layer "F.Cu") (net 14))
 (segment (start 85.09 91.44) (end 91.44 85.09) (width 0.25) (layer "F.Cu") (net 14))
 (segment (start 100.965 92.71) (end 100.335 92.71) (width 0.25) (layer "F.Cu") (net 5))
 (segment (start 116.84 92.71) (end 105.41 92.71) (width 0.25) (layer "F.Cu") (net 5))
 (segment (start 120.65 96.52) (end 116.84 92.71) (width 0.25) (layer "F.Cu") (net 5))
 (segment (start 100.335 92.71) (end 97.805 95.24) (width 0.25) (layer "F.Cu") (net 5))
 (via (at 100.965 92.71) (size 0.8) (drill 0.4) (layers "F.Cu" "B.Cu") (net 5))
 (via (at 105.41 92.71) (size 0.8) (drill 0.4) (layers "F.Cu" "B.Cu") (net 5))
 (segment (start 105.41 92.71) (end 100.965 92.71) (width 0.25) (layer "B.Cu") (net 5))
 (segment (start 123.19 100.33) (end 123.19 102.87) (width 0.25) (layer "F.Cu") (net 6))
 (segment (start 121.92 104.14) (end 109.245 104.14) (width 0.25) (layer "F.Cu") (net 6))
 (segment (start 109.245 104.14) (end 100.345 95.24) (width 0.25) (layer "F.Cu") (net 6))
 (segment (start 121.92 99.06) (end 123.19 100.33) (width 0.25) (layer "F.Cu") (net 6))
 (segment (start 123.19 102.87) (end 121.92 104.14) (width 0.25) (layer "F.Cu") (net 6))
 (segment (start 120.65 99.06) (end 121.92 99.06) (width 0.25) (layer "F.Cu") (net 6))
 (segment (start 101.625 91.44) (end 105.425 95.24) (width 0.25) (layer "F.Cu") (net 18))
 (segment (start 95.25 88.9) (end 97.79 91.44) (width 0.25) (layer "F.Cu") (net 18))
 (segment (start 92.71 88.9) (end 95.25 88.9) (width 0.25) (layer "F.Cu") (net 18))
 (segment (start 97.79 91.44) (end 101.625 91.44) (width 0.25) (layer "F.Cu") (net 18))
 (segment (start 93.345 104.775) (end 98.43 104.775) (width 0.25) (layer "B.Cu") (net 17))
 (segment (start 98.43 104.775) (end 107.965 95.24) (width 0.25) (layer "B.Cu") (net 17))
 (segment (start 85.09 96.52) (end 93.345 104.775) (width 0.25) (layer "B.Cu") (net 17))
 (segment (start 79.52 100.28) (end 79.47 100.33) (width 0.25) (layer "F.Cu") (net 22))
 (segment (start 79.52 97.79) (end 79.52 100.28) (width 0.25) (layer "F.Cu") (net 22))
 (segment (start 82.55 91.44) (end 85.09 93.98) (width 0.25) (layer "F.Cu") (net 2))
 (segment (start 123.19 92.71) (end 123.19 88.9) (width 0.25) (layer "F.Cu") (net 2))
 (segment (start 128.27 101.6) (end 127 101.6) (width 0.25) (layer "F.Cu") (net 2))
 (segment (start 85.09 86.36) (end 82.55 88.9) (width 0.25) (layer "F.Cu") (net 2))
 (segment (start 134.16 93.98) (end 137.16 90.98) (width 0.25) (layer "F.Cu") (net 2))
 (segment (start 128.27 93.98) (end 134.16 93.98) (width 0.25) (layer "F.Cu") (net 2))
 (segment (start 127 101.6) (end 125.73 100.33) (width 0.25) (layer "F.Cu") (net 2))
 (segment (start 120.65 93.98) (end 121.92 93.98) (width 0.25) (layer "F.Cu") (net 2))
 (segment (start 82.55 88.9) (end 82.55 91.44) (width 0.25) (layer "F.Cu") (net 2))
 (segment (start 123.19 88.9) (end 120.65 86.36) (width 0.25) (layer "F.Cu") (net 2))
 (segment (start 121.92 93.98) (end 123.19 92.71) (width 0.25) (layer "F.Cu") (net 2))
 (segment (start 125.73 100.33) (end 125.73 93.98) (width 0.25) (layer "F.Cu") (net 2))
 (segment (start 120.65 93.98) (end 125.73 93.98) (width 0.25) (layer "F.Cu") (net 2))
 (segment (start 125.73 93.98) (end 128.27 93.98) (width 0.25) (layer "F.Cu") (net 2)))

